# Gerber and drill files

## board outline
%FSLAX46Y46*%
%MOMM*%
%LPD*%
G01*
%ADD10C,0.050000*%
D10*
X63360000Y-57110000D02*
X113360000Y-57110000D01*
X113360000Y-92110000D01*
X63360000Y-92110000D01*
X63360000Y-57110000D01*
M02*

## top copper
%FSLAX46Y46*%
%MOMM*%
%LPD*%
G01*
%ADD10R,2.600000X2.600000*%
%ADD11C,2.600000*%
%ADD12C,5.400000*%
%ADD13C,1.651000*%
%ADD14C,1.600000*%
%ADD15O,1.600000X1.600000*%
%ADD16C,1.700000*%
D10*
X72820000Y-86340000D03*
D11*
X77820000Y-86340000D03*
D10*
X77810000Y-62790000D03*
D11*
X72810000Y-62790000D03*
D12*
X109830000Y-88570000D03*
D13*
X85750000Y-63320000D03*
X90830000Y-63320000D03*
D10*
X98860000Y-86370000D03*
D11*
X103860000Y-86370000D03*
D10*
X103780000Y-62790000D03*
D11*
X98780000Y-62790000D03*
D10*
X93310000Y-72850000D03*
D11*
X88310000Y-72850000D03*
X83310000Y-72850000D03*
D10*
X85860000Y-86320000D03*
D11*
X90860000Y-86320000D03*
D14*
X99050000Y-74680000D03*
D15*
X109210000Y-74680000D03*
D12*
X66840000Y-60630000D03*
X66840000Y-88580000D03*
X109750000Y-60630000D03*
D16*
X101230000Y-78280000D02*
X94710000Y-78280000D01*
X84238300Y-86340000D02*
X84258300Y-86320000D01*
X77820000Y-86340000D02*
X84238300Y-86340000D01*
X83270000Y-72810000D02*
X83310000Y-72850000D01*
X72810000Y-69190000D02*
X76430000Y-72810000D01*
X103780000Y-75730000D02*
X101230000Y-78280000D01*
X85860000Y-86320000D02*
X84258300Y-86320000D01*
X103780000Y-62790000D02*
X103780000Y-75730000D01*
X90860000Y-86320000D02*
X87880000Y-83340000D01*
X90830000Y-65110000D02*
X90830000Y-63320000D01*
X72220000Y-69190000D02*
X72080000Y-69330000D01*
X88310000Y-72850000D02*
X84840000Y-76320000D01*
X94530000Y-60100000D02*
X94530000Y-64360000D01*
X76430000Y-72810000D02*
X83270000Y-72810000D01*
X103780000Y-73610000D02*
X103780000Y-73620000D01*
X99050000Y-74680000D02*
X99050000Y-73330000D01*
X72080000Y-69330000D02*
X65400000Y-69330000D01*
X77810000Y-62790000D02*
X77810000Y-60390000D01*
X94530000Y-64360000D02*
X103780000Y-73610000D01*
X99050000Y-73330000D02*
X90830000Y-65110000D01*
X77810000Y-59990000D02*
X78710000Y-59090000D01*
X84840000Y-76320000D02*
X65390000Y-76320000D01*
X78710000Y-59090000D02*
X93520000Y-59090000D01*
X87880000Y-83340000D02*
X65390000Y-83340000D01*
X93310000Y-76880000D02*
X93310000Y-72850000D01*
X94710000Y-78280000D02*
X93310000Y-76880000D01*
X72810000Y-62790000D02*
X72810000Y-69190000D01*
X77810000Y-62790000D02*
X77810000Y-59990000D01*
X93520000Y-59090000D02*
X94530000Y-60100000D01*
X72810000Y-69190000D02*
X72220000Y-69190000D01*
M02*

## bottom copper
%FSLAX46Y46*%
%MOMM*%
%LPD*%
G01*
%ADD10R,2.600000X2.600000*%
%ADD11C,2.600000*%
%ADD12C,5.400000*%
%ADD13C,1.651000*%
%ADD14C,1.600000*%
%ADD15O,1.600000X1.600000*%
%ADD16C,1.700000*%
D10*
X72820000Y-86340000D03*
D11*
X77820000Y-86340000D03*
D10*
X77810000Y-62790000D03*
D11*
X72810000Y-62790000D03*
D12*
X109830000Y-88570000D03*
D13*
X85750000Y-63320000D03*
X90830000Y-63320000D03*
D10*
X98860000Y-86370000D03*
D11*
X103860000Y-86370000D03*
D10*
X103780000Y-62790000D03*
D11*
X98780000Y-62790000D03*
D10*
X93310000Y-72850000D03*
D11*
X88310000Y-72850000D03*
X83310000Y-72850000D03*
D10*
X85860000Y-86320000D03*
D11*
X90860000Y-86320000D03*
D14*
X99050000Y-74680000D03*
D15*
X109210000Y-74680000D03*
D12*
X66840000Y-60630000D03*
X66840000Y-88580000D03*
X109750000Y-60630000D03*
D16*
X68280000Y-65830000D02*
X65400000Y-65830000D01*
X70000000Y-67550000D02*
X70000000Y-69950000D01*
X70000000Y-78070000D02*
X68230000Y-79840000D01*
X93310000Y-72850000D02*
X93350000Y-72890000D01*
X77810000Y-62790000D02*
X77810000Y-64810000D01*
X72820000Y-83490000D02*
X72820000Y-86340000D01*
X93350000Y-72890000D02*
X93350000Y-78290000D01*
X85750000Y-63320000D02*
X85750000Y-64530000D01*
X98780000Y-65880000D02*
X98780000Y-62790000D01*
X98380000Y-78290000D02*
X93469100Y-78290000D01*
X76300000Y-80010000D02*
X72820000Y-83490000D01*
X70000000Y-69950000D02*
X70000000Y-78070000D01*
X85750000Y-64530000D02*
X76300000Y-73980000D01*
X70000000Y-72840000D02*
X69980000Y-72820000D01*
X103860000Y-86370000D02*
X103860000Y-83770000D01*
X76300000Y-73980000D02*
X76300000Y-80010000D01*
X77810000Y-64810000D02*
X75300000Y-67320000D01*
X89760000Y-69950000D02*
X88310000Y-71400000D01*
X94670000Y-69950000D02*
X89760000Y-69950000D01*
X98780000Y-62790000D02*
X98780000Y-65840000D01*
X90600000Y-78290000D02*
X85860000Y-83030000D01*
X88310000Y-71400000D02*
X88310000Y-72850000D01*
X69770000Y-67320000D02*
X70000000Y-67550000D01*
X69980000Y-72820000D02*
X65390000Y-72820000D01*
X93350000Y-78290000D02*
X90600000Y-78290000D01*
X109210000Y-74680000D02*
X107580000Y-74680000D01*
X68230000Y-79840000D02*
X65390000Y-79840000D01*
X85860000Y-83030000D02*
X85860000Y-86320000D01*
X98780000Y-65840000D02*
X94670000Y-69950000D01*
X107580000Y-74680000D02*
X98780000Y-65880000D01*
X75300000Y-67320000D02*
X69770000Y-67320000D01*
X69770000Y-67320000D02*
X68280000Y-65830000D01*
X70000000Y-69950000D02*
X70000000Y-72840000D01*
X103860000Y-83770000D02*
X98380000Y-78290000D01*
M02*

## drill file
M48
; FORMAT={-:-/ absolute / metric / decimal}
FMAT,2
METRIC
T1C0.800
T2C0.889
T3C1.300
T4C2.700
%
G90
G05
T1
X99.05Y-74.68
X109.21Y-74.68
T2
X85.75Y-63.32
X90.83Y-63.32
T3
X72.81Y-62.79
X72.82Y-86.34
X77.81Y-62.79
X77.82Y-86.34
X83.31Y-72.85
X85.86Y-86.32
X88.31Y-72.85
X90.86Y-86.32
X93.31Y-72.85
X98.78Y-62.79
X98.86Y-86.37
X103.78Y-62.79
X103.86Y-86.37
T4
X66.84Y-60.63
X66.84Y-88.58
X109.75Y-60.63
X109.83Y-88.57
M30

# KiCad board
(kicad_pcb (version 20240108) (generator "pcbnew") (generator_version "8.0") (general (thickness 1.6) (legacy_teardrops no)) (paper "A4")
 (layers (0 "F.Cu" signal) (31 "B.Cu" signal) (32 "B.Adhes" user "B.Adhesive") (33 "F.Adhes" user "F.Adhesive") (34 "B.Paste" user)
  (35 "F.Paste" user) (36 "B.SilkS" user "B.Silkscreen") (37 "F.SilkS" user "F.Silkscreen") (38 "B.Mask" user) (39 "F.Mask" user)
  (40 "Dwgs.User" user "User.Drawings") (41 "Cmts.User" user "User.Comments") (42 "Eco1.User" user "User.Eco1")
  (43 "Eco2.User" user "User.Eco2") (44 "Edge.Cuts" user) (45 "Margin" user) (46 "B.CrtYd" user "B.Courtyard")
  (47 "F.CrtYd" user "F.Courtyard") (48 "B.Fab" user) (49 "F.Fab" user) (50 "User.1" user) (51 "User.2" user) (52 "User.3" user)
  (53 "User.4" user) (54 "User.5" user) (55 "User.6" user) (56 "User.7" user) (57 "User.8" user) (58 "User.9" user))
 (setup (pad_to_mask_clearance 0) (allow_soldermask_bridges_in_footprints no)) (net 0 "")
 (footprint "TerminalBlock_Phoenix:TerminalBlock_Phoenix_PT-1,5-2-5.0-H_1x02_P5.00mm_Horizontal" (layer "F.Cu") (at 72.82 86.34)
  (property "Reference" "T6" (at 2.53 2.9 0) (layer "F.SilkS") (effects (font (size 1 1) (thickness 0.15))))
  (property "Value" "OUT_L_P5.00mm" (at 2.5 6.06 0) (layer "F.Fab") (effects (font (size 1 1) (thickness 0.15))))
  (pad "1" thru_hole rect (at 0 0) (size 2.6 2.6) (drill 1.3) (layers "*.Cu" "*.Mask") (remove_unused_layers no))
  (pad "2" thru_hole circle (at 5 0) (size 2.6 2.6) (drill 1.3) (layers "*.Cu" "*.Mask") (remove_unused_layers no)))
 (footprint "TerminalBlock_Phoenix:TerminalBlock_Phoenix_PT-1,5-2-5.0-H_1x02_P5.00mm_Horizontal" (layer "F.Cu") (at 77.81 62.79 180)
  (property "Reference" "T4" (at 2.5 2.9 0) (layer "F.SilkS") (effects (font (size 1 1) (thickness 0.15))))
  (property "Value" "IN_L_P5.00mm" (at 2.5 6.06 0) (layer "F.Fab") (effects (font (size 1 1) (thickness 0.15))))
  (pad "1" thru_hole rect (at 0 0 180) (size 2.6 2.6) (drill 1.3) (layers "*.Cu" "*.Mask") (remove_unused_layers no))
  (pad "2" thru_hole circle (at 5 0 180) (size 2.6 2.6) (drill 1.3) (layers "*.Cu" "*.Mask") (remove_unused_layers no)))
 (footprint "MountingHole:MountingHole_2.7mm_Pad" (layer "F.Cu") (at 109.83 88.57)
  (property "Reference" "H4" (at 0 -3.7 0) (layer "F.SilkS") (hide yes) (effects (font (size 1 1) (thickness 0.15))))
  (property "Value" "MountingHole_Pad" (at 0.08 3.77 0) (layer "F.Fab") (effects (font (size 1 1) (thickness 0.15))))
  (pad "1" thru_hole circle (at 0 0) (size 5.4 5.4) (drill 2.7) (layers "*.Cu" "*.Mask") (remove_unused_layers no)))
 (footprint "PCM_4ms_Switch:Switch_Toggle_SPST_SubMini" (layer "F.Cu") (at 88.29 63.32 90)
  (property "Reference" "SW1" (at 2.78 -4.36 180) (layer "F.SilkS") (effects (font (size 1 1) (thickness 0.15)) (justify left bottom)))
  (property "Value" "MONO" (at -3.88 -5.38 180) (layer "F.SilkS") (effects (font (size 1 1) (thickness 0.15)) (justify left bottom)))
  (pad "1" thru_hole circle (at 0 -2.54 90) (size 1.651 1.651) (drill 0.889) (layers "*.Cu" "*.Mask") (remove_unused_layers no))
  (pad "2" thru_hole circle (at 0 2.54 90) (size 1.651 1.651) (drill 0.889) (layers "*.Cu" "*.Mask") (remove_unused_layers no)))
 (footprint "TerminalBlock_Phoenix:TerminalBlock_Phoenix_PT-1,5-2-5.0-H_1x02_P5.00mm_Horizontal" (layer "F.Cu") (at 98.86 86.37)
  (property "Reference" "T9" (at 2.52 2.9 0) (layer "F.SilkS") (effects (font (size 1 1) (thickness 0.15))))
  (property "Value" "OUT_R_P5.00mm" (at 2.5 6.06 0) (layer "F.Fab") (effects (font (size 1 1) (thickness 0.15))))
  (pad "1" thru_hole rect (at 0 0) (size 2.6 2.6) (drill 1.3) (layers "*.Cu" "*.Mask") (remove_unused_layers no))
  (pad "2" thru_hole circle (at 5 0) (size 2.6 2.6) (drill 1.3) (layers "*.Cu" "*.Mask") (remove_unused_layers no)))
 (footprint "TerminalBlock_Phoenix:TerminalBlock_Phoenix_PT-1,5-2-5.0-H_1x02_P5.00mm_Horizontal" (layer "F.Cu") (at 103.78 62.79 180)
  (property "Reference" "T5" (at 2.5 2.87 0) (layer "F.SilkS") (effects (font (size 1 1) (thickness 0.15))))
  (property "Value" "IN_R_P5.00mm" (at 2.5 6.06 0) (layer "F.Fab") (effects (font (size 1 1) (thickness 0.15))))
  (pad "1" thru_hole rect (at 0 0 180) (size 2.6 2.6) (drill 1.3) (layers "*.Cu" "*.Mask") (remove_unused_layers no))
  (pad "2" thru_hole circle (at 5 0 180) (size 2.6 2.6) (drill 1.3) (layers "*.Cu" "*.Mask") (remove_unused_layers no)))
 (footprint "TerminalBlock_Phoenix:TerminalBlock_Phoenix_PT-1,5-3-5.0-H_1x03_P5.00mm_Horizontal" (layer "F.Cu") (at 93.31 72.85 180)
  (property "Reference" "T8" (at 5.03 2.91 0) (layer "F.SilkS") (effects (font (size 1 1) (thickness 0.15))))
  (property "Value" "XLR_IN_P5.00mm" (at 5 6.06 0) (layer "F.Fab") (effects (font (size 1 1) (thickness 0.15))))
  (pad "1" thru_hole rect (at 0 0 180) (size 2.6 2.6) (drill 1.3) (layers "*.Cu" "*.Mask") (remove_unused_layers no))
  (pad "2" thru_hole circle (at 5 0 180) (size 2.6 2.6) (drill 1.3) (layers "*.Cu" "*.Mask") (remove_unused_layers no))
  (pad "3" thru_hole circle (at 10 0 180) (size 2.6 2.6) (drill 1.3) (layers "*.Cu" "*.Mask") (remove_unused_layers no)))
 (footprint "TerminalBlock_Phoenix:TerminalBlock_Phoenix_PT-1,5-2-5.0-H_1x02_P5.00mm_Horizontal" (layer "F.Cu") (at 85.86 86.32)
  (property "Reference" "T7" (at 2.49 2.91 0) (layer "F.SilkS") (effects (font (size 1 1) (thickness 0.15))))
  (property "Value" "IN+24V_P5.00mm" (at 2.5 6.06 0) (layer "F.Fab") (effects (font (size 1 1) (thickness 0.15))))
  (pad "1" thru_hole rect (at 0 0) (size 2.6 2.6) (drill 1.3) (layers "*.Cu" "*.Mask") (remove_unused_layers no))
  (pad "2" thru_hole circle (at 5 0) (size 2.6 2.6) (drill 1.3) (layers "*.Cu" "*.Mask") (remove_unused_layers no)))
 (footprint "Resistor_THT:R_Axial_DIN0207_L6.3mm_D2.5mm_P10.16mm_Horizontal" (layer "F.Cu") (at 99.05 74.68)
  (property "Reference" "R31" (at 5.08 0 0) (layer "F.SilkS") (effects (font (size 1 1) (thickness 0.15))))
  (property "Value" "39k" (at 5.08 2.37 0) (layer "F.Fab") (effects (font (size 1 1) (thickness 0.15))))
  (pad "1" thru_hole circle (at 0 0) (size 1.6 1.6) (drill 0.8) (layers "*.Cu" "*.Mask") (remove_unused_layers no))
  (pad "2" thru_hole oval (at 10.16 0) (size 1.6 1.6) (drill 0.8) (layers "*.Cu" "*.Mask") (remove_unused_layers no)))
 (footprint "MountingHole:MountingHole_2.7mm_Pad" (layer "F.Cu") (at 66.84 60.63)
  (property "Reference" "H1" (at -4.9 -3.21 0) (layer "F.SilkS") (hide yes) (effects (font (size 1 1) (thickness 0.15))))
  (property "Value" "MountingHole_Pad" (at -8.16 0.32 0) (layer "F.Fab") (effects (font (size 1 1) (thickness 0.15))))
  (pad "1" thru_hole circle (at 0 0) (size 5.4 5.4) (drill 2.7) (layers "*.Cu" "*.Mask") (remove_unused_layers no)))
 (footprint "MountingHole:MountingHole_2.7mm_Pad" (layer "F.Cu") (at 66.84 88.58)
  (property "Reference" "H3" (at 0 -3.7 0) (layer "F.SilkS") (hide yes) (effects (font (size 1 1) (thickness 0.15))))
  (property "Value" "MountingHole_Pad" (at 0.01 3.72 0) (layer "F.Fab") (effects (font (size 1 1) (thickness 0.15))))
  (pad "1" thru_hole circle (at 0 0) (size 5.4 5.4) (drill 2.7) (layers "*.Cu" "*.Mask") (remove_unused_layers no)))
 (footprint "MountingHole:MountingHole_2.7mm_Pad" (layer "F.Cu") (at 109.75 60.63)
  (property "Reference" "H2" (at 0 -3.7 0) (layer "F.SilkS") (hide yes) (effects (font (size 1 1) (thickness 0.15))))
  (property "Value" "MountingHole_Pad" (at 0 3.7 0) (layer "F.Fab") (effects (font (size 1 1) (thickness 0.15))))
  (pad "1" thru_hole circle (at 0 0) (size 5.4 5.4) (drill 2.7) (layers "*.Cu" "*.Mask") (remove_unused_layers no)))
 (gr_rect (start 63.36 57.11) (end 113.36 92.11) (stroke (width 0.05) (type default)) (fill none) (layer "Edge.Cuts"))
 (segment (start 101.23 78.28) (end 94.71 78.28) (width 1.7) (layer "F.Cu") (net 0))
 (segment (start 84.2383 86.34) (end 84.2583 86.32) (width 1.7) (layer "F.Cu") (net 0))
 (segment (start 77.82 86.34) (end 84.2383 86.34) (width 1.7) (layer "F.Cu") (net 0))
 (segment (start 83.27 72.81) (end 83.31 72.85) (width 1.7) (layer "F.Cu") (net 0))
 (segment (start 72.81 69.19) (end 76.43 72.81) (width 1.7) (layer "F.Cu") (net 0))
 (segment (start 103.78 75.73) (end 101.23 78.28) (width 1.7) (layer "F.Cu") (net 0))
 (segment (start 85.86 86.32) (end 84.2583 86.32) (width 1.7) (layer "F.Cu") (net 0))
 (segment (start 103.78 62.79) (end 103.78 75.73) (width 1.7) (layer "F.Cu") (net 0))
 (segment (start 90.86 86.32) (end 87.88 83.34) (width 1.7) (layer "F.Cu") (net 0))
 (segment (start 90.83 65.11) (end 90.83 63.32) (width 1.7) (layer "F.Cu") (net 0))
 (segment (start 72.22 69.19) (end 72.08 69.33) (width 1.7) (layer "F.Cu") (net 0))
 (segment (start 88.31 72.85) (end 84.84 76.32) (width 1.7) (layer "F.Cu") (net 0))
 (segment (start 94.53 60.1) (end 94.53 64.36) (width 1.7) (layer "F.Cu") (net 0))
 (segment (start 76.43 72.81) (end 83.27 72.81) (width 1.7) (layer "F.Cu") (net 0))
 (segment (start 103.78 73.61) (end 103.78 73.62) (width 1.7) (layer "F.Cu") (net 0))
 (segment (start 99.05 74.68) (end 99.05 73.33) (width 1.7) (layer "F.Cu") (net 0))
 (segment (start 72.08 69.33) (end 65.4 69.33) (width 1.7) (layer "F.Cu") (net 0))
 (segment (start 77.81 62.79) (end 77.81 60.39) (width 1.7) (layer "F.Cu") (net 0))
 (segment (start 94.53 64.36) (end 103.78 73.61) (width 1.7) (layer "F.Cu") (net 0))
 (segment (start 99.05 73.33) (end 90.83 65.11) (width 1.7) (layer "F.Cu") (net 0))
 (segment (start 77.81 59.99) (end 78.71 59.09) (width 1.7) (layer "F.Cu") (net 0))
 (segment (start 84.84 76.32) (end 65.39 76.32) (width 1.7) (layer "F.Cu") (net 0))
 (segment (start 78.71 59.09) (end 93.52 59.09) (width 1.7) (layer "F.Cu") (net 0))
 (segment (start 87.88 83.34) (end 65.39 83.34) (width 1.7) (layer "F.Cu") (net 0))
 (segment (start 93.31 76.88) (end 93.31 72.85) (width 1.7) (layer "F.Cu") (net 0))
 (segment (start 94.71 78.28) (end 93.31 76.88) (width 1.7) (layer "F.Cu") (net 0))
 (segment (start 72.81 62.79) (end 72.81 69.19) (width 1.7) (layer "F.Cu") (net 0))
 (segment (start 77.81 62.79) (end 77.81 59.99) (width 1.7) (layer "F.Cu") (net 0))
 (segment (start 93.52 59.09) (end 94.53 60.1) (width 1.7) (layer "F.Cu") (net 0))
 (segment (start 72.81 69.19) (end 72.22 69.19) (width 1.7) (layer "F.Cu") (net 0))
 (segment (start 68.28 65.83) (end 65.4 65.83) (width 1.7) (layer "B.Cu") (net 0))
 (segment (start 70 67.55) (end 70 69.95) (width 1.7) (layer "B.Cu") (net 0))
 (segment (start 70 78.07) (end 68.23 79.84) (width 1.7) (layer "B.Cu") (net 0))
 (segment (start 93.31 72.85) (end 93.35 72.89) (width 1.7) (layer "B.Cu") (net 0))
 (segment (start 77.81 62.79) (end 77.81 64.81) (width 1.7) (layer "B.Cu") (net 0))
 (segment (start 72.82 83.49) (end 72.82 86.34) (width 1.7) (layer "B.Cu") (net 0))
 (segment (start 93.35 72.89) (end 93.35 78.29) (width 1.7) (layer "B.Cu") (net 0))
 (segment (start 85.75 63.32) (end 85.75 64.53) (width 1.7) (layer "B.Cu") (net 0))
 (segment (start 98.78 65.88) (end 98.78 62.79) (width 1.7) (layer "B.Cu") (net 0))
 (segment (start 98.38 78.29) (end 93.4691 78.29) (width 1.7) (layer "B.Cu") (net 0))
 (segment (start 76.3 80.01) (end 72.82 83.49) (width 1.7) (layer "B.Cu") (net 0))
 (segment (start 70 69.95) (end 70 78.07) (width 1.7) (layer "B.Cu") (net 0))
 (segment (start 85.75 64.53) (end 76.3 73.98) (width 1.7) (layer "B.Cu") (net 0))
 (segment (start 70 72.84) (end 69.98 72.82) (width 1.7) (layer "B.Cu") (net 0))
 (segment (start 103.86 86.37) (end 103.86 83.77) (width 1.7) (layer "B.Cu") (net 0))
 (segment (start 76.3 73.98) (end 76.3 80.01) (width 1.7) (layer "B.Cu") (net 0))
 (segment (start 77.81 64.81) (end 75.3 67.32) (width 1.7) (layer "B.Cu") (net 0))
 (segment (start 89.76 69.95) (end 88.31 71.4) (width 1.7) (layer "B.Cu") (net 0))
 (segment (start 94.67 69.95) (end 89.76 69.95) (width 1.7) (layer "B.Cu") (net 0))
 (segment (start 98.78 62.79) (end 98.78 65.84) (width 1.7) (layer "B.Cu") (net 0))
 (segment (start 90.6 78.29) (end 85.86 83.03) (width 1.7) (layer "B.Cu") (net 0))
 (segment (start 88.31 71.4) (end 88.31 72.85) (width 1.7) (layer "B.Cu") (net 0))
 (segment (start 69.77 67.32) (end 70 67.55) (width 1.7) (layer "B.Cu") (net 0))
 (segment (start 69.98 72.82) (end 65.39 72.82) (width 1.7) (layer "B.Cu") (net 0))
 (segment (start 93.35 78.29) (end 90.6 78.29) (width 1.7) (layer "B.Cu") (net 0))
 (segment (start 109.21 74.68) (end 107.58 74.68) (width 1.7) (layer "B.Cu") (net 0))
 (segment (start 68.23 79.84) (end 65.39 79.84) (width 1.7) (layer "B.Cu") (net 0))
 (segment (start 85.86 83.03) (end 85.86 86.32) (width 1.7) (layer "B.Cu") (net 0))
 (segment (start 98.78 65.84) (end 94.67 69.95) (width 1.7) (layer "B.Cu") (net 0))
 (segment (start 107.58 74.68) (end 98.78 65.88) (width 1.7) (layer "B.Cu") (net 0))
 (segment (start 75.3 67.32) (end 69.77 67.32) (width 1.7) (layer "B.Cu") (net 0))
 (segment (start 69.77 67.32) (end 68.28 65.83) (width 1.7) (layer "B.Cu") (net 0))
 (segment (start 70 69.95) (end 70 72.84) (width 1.7) (layer "B.Cu") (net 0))
 (segment (start 103.86 83.77) (end 98.38 78.29) (width 1.7) (layer "B.Cu") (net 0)))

